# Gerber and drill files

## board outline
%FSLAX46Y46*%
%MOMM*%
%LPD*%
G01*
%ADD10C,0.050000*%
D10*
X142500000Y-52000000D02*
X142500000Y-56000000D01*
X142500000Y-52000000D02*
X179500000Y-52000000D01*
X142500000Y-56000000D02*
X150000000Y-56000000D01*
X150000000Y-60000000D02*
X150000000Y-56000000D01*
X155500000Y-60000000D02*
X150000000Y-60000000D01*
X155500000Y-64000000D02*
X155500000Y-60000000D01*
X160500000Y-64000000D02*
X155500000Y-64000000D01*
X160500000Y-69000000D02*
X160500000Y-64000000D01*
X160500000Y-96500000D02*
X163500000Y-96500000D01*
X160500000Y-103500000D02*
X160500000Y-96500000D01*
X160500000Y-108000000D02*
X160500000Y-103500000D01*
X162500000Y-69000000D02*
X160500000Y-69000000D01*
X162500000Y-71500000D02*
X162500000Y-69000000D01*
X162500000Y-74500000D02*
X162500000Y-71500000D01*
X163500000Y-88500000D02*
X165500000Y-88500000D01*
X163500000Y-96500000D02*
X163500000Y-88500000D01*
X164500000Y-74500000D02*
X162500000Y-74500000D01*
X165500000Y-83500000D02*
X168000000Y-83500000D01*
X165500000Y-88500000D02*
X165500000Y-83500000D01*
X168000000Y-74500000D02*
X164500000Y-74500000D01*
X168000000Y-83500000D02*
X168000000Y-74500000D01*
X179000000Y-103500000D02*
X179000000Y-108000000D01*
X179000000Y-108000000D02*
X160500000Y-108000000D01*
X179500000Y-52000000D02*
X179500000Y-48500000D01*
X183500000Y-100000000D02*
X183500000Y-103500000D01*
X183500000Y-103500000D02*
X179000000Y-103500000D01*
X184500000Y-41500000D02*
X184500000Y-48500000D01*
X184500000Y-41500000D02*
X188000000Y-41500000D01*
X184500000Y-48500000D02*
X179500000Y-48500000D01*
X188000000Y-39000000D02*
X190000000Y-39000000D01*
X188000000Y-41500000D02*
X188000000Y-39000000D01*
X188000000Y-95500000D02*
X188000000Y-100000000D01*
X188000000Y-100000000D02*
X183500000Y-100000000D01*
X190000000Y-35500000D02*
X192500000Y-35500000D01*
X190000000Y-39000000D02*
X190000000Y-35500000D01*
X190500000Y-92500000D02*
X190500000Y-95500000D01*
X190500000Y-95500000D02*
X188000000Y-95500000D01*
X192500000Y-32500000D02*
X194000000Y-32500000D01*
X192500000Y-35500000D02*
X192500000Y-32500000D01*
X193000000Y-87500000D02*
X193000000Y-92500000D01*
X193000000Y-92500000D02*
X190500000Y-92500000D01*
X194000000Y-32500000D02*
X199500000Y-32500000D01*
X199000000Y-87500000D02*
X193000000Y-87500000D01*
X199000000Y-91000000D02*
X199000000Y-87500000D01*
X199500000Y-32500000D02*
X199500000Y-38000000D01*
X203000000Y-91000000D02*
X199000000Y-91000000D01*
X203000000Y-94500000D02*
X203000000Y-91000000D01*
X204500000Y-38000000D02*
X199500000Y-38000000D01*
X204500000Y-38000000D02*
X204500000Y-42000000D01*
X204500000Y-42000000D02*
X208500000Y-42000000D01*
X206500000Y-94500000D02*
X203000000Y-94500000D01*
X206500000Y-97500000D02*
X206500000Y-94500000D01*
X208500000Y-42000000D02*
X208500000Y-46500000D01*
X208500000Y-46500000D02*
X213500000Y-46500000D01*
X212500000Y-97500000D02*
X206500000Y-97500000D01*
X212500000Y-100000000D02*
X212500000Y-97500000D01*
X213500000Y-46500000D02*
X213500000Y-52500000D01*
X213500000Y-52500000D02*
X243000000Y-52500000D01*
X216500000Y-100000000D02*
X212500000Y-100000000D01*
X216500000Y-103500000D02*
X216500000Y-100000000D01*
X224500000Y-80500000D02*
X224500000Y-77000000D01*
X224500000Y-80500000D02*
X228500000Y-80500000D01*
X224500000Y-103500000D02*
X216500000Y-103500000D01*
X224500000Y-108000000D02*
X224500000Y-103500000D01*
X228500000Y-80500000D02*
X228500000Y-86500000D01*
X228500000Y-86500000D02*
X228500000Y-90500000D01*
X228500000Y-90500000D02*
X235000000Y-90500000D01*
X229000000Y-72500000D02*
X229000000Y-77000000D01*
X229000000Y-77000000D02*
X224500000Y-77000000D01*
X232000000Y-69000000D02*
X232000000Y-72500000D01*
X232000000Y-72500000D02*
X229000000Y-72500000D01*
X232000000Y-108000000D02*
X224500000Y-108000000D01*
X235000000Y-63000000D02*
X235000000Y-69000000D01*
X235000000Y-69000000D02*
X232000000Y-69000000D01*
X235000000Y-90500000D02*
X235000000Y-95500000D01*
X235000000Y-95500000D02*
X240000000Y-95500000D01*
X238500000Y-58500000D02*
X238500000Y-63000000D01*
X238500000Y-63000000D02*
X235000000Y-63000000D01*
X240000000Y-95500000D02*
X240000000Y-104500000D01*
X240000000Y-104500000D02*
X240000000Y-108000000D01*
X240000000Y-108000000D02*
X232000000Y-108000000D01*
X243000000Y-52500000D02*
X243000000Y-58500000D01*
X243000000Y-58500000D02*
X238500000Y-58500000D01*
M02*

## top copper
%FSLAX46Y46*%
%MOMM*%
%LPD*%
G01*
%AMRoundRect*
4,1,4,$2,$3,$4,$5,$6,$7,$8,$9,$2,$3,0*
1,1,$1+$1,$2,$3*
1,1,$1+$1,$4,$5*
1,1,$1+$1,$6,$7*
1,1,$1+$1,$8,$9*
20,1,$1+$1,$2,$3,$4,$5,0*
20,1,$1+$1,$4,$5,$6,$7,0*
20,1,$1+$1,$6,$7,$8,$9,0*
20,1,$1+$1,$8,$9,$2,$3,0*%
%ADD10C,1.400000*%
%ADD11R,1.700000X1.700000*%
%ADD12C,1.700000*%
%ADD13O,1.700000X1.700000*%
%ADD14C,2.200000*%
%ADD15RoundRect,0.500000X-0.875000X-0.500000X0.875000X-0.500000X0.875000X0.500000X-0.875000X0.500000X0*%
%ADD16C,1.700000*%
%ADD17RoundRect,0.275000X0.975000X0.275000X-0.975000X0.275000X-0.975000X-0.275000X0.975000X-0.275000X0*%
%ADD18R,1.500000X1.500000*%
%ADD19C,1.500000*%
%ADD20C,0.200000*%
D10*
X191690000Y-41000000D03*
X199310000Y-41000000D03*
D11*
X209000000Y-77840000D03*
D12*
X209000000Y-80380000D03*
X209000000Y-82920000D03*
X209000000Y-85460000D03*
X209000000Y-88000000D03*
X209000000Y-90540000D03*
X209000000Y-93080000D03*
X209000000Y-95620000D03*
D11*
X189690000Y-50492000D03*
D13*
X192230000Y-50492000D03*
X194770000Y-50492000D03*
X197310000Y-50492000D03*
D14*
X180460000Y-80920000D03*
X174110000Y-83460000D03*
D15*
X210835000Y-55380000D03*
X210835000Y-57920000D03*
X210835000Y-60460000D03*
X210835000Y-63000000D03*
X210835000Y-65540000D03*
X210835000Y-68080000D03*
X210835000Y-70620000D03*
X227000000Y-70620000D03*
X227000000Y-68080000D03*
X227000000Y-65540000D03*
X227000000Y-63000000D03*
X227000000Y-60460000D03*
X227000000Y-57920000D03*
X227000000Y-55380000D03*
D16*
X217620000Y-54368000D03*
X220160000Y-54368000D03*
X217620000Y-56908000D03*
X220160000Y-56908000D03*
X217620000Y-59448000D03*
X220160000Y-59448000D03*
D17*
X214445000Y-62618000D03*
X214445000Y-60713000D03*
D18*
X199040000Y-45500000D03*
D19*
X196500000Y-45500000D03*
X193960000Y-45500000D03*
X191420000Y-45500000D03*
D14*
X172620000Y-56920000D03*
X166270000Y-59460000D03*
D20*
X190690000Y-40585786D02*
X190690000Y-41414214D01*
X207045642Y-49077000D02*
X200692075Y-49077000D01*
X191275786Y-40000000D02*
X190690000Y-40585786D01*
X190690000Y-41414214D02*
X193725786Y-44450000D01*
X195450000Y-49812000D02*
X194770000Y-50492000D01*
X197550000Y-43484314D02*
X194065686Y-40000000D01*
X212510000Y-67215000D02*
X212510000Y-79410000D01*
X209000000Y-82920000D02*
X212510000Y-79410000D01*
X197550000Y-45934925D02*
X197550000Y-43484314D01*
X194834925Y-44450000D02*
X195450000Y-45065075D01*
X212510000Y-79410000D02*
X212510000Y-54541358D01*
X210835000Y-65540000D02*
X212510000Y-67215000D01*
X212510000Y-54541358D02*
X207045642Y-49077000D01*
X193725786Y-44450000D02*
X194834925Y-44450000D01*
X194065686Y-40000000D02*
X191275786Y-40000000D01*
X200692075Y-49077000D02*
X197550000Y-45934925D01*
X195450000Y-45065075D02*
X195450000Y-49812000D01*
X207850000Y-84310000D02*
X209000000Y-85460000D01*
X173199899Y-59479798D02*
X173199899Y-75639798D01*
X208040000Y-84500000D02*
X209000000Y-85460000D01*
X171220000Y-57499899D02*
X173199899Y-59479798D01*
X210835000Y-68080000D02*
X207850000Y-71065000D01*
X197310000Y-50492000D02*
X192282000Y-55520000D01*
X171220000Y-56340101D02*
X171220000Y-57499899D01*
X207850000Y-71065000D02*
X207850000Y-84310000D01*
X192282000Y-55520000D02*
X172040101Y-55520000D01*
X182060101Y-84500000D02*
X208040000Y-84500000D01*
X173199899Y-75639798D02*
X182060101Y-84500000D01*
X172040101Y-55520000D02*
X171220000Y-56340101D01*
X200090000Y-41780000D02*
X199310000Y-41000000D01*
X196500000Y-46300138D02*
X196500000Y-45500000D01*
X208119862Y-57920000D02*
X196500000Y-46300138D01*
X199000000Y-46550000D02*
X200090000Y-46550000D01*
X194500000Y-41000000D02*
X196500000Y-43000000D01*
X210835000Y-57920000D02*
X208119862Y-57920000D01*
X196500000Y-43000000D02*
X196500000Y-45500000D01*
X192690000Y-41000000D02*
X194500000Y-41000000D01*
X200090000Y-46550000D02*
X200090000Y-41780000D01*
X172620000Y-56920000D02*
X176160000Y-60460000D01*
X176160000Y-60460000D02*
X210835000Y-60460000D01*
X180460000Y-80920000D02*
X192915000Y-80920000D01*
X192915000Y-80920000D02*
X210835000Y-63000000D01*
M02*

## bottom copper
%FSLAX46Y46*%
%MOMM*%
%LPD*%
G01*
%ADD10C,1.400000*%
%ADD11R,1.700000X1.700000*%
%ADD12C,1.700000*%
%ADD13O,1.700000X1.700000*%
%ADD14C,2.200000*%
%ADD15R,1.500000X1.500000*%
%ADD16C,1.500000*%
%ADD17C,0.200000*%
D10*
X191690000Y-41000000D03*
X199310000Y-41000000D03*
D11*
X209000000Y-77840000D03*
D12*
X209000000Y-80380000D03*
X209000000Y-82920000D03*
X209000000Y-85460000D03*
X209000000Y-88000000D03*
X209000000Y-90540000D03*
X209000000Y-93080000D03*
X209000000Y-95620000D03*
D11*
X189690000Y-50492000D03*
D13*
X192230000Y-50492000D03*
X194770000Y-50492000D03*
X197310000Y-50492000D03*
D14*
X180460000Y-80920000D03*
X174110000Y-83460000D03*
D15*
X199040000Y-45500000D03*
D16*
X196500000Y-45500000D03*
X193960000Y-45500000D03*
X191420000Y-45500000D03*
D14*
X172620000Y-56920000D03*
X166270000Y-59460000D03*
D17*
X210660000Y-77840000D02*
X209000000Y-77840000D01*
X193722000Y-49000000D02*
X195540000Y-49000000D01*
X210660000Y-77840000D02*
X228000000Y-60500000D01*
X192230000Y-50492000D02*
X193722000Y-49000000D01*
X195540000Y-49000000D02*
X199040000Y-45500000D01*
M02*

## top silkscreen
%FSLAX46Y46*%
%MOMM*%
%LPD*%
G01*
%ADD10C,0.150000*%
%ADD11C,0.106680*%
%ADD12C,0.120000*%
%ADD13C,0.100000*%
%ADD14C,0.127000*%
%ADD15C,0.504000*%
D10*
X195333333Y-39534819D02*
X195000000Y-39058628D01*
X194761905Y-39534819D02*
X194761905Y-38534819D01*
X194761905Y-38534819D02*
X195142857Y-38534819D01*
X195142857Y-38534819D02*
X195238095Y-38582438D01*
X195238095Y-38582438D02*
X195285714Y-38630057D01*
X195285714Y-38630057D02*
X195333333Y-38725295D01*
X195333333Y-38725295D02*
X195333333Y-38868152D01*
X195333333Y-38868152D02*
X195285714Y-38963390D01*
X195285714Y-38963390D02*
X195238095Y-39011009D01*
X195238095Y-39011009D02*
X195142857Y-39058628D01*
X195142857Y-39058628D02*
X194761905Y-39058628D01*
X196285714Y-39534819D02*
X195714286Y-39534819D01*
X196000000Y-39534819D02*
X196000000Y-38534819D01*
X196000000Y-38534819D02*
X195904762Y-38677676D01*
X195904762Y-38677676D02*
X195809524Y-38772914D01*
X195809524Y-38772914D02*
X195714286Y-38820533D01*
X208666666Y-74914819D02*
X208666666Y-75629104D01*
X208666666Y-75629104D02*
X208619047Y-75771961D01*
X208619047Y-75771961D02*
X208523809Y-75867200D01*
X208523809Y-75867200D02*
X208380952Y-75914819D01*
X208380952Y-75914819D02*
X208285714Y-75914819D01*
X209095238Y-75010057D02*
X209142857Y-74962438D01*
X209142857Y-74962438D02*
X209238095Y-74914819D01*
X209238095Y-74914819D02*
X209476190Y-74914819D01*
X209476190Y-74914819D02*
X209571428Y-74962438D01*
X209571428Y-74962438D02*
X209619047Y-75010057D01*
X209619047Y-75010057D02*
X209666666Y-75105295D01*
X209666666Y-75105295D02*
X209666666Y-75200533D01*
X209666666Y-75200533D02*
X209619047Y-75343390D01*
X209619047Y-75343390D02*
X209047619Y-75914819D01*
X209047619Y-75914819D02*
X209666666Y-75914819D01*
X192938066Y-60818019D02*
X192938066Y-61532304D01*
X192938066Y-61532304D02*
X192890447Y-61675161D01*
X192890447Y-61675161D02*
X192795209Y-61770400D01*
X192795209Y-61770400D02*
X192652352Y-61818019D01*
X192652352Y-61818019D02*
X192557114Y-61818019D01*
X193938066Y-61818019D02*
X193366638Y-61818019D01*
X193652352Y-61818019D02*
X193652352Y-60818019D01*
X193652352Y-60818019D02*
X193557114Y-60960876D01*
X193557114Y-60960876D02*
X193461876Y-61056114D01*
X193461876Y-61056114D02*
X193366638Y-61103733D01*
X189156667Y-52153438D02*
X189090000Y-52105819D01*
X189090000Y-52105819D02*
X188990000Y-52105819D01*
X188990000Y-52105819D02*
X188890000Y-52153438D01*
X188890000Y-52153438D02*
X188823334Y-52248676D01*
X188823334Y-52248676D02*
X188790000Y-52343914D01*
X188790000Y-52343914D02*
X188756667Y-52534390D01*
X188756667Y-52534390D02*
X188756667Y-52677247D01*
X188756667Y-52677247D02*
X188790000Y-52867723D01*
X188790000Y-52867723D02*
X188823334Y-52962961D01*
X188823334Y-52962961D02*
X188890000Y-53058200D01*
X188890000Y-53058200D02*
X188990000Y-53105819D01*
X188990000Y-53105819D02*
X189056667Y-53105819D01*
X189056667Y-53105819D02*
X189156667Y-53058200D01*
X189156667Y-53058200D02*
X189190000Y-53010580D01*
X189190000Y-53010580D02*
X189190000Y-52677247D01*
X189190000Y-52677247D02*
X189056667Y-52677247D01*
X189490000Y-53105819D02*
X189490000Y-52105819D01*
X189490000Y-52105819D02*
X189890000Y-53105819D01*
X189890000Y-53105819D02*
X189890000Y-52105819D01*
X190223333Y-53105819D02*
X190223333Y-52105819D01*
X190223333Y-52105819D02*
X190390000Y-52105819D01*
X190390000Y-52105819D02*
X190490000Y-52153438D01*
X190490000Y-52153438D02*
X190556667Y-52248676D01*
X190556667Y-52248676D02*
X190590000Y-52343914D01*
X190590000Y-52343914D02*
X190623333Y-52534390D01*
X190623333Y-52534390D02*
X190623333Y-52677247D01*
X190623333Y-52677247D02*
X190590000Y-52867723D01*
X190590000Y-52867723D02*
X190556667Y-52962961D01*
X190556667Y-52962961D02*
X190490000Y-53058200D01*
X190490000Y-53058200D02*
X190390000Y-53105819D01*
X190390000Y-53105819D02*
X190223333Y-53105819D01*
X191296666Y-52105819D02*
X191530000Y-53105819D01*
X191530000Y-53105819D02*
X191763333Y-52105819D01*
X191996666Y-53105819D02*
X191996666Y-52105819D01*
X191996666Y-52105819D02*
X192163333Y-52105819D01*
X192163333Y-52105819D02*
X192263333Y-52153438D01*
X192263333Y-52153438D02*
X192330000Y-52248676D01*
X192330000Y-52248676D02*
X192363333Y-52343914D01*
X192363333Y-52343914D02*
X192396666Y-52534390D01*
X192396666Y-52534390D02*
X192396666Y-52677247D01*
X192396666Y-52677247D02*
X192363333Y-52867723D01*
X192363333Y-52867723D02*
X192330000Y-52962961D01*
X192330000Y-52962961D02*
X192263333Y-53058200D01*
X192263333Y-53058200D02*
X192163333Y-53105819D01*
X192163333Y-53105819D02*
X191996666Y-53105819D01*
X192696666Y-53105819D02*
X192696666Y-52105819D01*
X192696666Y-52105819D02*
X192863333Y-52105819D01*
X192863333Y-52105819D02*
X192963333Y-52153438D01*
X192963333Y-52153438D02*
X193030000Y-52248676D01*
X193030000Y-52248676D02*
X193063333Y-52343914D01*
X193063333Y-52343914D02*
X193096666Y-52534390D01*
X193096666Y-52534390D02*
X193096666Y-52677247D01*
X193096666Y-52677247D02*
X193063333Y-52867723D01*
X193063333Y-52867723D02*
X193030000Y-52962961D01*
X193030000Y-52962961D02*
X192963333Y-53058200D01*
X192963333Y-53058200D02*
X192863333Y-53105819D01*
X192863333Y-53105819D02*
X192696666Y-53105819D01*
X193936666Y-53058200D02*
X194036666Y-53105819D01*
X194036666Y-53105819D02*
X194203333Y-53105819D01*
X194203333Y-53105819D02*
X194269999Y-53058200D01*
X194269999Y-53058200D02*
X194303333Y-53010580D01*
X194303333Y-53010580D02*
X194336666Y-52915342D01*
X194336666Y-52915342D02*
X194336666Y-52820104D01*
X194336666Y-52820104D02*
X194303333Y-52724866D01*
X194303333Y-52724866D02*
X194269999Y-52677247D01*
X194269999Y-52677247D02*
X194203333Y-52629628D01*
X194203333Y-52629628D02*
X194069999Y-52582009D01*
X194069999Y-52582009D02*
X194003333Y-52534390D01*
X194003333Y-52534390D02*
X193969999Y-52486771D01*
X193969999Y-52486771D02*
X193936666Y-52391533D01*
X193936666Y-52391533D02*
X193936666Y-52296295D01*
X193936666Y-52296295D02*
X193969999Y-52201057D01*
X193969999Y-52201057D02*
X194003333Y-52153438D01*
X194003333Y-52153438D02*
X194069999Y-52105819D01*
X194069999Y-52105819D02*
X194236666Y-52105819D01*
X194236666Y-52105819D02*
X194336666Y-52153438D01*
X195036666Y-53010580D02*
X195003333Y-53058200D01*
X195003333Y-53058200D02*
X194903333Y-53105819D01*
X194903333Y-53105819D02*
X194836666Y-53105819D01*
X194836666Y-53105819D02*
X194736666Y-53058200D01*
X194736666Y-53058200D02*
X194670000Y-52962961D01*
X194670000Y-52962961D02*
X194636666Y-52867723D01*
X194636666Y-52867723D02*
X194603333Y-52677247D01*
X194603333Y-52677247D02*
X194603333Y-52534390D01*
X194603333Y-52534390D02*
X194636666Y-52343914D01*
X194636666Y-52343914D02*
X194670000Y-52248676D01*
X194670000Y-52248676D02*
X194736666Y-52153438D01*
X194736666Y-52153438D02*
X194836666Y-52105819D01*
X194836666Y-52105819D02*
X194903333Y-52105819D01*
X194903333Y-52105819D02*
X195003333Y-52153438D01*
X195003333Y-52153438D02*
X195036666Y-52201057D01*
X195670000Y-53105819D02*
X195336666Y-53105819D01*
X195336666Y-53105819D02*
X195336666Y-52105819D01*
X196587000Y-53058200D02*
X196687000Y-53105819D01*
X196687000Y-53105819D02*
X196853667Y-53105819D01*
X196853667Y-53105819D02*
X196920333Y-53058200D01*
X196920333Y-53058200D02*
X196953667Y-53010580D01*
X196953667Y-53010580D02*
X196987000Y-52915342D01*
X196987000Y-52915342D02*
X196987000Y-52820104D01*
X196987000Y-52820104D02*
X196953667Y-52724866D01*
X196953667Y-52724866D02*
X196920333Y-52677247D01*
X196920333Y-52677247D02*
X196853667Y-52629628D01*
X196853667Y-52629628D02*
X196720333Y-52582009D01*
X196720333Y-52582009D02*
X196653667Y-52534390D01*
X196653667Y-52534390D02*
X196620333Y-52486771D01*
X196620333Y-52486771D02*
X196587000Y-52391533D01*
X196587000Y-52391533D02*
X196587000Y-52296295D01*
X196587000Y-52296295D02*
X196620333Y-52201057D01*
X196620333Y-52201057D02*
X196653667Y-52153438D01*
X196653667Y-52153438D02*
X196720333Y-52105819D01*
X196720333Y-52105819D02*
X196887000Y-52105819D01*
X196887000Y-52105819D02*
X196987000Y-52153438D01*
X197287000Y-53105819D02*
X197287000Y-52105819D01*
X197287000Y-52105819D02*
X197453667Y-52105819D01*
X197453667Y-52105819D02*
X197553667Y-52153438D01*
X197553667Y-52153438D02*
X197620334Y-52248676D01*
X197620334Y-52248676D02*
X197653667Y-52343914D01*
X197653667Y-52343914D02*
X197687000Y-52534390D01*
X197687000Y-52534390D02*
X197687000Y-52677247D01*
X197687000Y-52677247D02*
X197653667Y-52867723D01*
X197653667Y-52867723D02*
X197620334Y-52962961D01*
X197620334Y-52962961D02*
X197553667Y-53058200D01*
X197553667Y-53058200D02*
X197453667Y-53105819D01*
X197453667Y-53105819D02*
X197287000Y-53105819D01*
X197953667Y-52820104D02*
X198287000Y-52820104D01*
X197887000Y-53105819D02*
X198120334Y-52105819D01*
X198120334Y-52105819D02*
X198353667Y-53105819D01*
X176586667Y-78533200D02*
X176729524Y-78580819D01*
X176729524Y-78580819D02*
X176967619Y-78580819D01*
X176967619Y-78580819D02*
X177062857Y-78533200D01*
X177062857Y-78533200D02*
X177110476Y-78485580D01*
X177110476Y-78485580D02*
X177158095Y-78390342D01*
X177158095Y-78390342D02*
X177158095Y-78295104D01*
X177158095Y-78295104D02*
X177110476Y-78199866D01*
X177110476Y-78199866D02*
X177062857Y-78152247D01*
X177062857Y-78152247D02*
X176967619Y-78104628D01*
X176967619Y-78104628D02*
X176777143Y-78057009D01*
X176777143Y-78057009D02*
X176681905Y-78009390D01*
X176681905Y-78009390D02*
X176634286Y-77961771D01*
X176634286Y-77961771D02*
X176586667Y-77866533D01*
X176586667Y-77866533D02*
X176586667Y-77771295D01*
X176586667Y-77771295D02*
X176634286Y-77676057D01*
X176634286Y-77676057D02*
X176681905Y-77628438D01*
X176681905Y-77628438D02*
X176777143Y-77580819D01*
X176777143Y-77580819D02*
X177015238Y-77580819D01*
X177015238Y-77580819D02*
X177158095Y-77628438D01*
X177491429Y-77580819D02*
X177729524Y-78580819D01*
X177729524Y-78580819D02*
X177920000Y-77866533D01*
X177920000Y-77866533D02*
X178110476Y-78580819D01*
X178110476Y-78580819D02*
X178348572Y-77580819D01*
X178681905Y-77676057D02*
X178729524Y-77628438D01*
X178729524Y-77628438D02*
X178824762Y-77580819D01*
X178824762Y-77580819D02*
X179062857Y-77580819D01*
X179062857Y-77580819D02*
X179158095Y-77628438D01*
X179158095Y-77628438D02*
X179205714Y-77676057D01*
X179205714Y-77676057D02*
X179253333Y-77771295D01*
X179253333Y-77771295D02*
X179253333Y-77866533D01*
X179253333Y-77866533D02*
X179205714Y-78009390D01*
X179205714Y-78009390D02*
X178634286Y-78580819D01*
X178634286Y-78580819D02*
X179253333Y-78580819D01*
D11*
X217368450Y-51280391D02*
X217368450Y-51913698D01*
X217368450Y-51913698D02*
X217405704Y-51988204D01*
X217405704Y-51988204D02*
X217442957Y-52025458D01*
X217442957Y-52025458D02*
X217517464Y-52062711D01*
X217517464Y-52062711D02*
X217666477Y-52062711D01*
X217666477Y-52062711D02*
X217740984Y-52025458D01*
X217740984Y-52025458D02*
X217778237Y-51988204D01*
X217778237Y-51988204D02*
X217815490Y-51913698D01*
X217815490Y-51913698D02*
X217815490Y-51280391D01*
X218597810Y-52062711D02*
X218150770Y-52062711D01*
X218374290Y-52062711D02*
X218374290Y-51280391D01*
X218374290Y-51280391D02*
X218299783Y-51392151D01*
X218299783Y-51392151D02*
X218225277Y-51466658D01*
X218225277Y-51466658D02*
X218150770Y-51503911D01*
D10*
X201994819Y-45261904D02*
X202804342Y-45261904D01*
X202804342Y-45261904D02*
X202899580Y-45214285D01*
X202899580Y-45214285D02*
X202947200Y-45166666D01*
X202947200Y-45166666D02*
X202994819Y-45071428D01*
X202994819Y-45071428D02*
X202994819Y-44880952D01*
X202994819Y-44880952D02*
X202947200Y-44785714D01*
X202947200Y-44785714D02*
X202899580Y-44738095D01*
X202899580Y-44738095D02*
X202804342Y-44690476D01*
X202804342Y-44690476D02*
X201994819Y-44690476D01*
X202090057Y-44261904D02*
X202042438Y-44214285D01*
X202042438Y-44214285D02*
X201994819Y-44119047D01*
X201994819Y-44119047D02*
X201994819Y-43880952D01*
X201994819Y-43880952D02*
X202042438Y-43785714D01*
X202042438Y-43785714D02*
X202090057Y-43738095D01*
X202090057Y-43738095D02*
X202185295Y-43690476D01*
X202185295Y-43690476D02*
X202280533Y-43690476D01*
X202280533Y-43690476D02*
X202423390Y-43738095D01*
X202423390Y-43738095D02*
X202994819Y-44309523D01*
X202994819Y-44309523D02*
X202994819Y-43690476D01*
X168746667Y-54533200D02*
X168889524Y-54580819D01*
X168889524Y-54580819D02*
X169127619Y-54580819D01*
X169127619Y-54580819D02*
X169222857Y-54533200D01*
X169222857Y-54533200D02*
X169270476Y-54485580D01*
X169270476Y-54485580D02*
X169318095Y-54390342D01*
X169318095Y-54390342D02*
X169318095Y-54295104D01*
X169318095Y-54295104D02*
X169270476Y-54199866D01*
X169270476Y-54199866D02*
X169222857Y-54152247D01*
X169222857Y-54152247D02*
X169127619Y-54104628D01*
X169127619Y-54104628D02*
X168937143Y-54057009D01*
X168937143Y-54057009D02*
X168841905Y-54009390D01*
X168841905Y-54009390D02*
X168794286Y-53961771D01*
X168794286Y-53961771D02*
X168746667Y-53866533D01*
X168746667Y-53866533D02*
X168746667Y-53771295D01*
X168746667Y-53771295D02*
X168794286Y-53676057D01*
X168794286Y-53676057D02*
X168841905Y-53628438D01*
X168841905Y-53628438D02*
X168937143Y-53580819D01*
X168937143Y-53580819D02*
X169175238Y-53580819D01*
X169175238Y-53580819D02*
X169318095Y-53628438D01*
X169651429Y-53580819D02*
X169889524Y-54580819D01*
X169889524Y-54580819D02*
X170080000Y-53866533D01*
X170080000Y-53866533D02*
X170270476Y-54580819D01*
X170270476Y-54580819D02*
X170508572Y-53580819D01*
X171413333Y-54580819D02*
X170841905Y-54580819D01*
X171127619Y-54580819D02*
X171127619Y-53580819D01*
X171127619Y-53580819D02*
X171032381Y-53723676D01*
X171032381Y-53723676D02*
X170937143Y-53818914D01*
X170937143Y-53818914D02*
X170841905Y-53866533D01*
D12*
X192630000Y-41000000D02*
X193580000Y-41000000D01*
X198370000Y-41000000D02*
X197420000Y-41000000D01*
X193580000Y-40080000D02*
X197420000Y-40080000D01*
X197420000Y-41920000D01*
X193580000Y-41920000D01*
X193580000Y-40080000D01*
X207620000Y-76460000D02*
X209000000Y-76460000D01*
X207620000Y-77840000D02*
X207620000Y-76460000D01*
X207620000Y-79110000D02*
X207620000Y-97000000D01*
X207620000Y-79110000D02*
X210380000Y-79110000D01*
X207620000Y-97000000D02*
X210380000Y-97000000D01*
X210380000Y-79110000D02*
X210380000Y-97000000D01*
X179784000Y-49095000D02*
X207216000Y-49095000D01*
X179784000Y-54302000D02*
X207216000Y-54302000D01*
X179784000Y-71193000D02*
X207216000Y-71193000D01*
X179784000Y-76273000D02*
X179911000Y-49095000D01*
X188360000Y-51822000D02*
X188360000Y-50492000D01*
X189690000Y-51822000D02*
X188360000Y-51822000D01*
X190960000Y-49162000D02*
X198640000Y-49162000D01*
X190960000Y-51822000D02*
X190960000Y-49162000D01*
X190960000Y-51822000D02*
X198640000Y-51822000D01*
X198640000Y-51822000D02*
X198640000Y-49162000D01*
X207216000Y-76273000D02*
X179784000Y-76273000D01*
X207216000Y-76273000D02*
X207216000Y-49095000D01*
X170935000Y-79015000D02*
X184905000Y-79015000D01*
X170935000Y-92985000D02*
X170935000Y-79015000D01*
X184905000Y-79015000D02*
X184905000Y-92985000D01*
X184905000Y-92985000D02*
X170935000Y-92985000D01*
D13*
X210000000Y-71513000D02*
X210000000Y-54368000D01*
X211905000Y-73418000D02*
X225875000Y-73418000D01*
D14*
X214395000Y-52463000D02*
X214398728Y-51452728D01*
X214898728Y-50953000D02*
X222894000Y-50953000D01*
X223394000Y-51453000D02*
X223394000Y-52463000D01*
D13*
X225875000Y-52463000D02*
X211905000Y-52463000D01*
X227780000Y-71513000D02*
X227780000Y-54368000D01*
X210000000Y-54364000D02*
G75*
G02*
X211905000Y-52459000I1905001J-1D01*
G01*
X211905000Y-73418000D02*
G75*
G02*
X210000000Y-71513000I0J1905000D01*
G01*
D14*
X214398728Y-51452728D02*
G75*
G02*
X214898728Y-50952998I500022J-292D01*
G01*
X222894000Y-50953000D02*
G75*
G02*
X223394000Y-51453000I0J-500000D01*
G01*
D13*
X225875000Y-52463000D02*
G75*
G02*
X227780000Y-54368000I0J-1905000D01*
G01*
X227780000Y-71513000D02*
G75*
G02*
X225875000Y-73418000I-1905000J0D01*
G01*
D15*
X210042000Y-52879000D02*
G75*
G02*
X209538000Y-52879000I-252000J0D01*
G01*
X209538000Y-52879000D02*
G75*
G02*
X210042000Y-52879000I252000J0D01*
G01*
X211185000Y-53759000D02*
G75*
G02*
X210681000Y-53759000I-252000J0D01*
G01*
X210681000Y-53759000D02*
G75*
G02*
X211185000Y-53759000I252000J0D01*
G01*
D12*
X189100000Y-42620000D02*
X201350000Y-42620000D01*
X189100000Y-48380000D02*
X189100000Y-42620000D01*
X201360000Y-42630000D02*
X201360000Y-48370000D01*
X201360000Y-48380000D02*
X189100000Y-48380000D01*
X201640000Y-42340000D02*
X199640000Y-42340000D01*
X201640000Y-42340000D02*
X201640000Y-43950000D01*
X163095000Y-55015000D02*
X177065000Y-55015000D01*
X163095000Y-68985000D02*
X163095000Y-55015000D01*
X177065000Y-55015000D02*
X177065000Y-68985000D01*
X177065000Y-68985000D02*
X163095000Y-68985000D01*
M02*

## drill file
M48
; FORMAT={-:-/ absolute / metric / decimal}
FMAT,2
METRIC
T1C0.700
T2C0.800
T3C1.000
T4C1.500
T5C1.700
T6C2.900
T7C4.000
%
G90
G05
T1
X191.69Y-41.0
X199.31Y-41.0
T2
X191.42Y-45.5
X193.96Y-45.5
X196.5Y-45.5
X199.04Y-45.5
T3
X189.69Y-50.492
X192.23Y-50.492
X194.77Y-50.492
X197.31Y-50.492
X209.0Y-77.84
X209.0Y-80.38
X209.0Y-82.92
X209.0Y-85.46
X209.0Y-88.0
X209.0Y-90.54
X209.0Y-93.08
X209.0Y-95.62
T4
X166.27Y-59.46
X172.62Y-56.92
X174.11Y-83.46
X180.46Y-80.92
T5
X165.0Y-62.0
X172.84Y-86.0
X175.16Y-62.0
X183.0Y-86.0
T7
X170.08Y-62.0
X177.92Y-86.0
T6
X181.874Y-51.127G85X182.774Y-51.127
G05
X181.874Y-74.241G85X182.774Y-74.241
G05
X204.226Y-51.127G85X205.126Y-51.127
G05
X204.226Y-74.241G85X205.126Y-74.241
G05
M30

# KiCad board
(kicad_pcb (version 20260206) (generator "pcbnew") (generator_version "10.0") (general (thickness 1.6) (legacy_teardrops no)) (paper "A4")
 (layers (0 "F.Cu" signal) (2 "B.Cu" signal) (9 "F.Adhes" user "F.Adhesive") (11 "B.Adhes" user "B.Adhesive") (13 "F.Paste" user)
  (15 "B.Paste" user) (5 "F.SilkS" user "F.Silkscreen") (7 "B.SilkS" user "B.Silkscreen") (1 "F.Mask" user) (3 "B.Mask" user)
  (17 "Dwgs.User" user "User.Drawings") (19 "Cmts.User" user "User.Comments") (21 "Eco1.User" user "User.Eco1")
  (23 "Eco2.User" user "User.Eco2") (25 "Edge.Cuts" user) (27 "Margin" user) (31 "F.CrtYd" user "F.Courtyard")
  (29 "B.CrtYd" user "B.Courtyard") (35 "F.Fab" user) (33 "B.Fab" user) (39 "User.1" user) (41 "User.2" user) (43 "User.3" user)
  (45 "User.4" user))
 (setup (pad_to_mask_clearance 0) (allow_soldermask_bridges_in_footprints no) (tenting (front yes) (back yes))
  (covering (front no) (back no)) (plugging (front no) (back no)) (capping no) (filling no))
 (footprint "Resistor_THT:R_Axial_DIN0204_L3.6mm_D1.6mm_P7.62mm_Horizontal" (layer "F.Cu") (at 191.69 41)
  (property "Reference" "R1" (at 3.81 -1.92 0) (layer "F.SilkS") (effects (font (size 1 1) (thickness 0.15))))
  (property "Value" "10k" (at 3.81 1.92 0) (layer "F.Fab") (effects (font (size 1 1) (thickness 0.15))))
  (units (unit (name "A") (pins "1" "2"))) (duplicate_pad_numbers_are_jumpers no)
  (fp_line (start 0.94 0) (end 1.89 0) (stroke (width 0.12) (type solid)) (layer "F.SilkS"))
  (fp_line (start 6.68 0) (end 5.73 0) (stroke (width 0.12) (type solid)) (layer "F.SilkS"))
  (fp_rect (start 1.89 -0.92) (end 5.73 0.92) (stroke (width 0.12) (type solid)) (fill no) (layer "F.SilkS"))
  (pad "1" thru_hole circle (at 0 0) (size 1.4 1.4) (drill 0.7) (layers "*.Cu" "*.Mask") (remove_unused_layers no) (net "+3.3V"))
  (pad "2" thru_hole circle (at 7.62 0) (size 1.4 1.4) (drill 0.7) (layers "*.Cu" "*.Mask") (remove_unused_layers no) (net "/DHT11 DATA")))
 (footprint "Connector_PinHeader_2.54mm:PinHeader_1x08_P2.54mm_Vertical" (layer "F.Cu") (at 209 77.84)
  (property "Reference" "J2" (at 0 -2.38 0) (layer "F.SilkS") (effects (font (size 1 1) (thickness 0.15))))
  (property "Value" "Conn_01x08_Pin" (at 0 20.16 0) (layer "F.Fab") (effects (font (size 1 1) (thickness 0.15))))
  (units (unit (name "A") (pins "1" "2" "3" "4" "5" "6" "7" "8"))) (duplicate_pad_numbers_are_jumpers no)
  (fp_line (start -1.38 -1.38) (end 0 -1.38) (stroke (width 0.12) (type solid)) (layer "F.SilkS"))
  (fp_line (start -1.38 0) (end -1.38 -1.38) (stroke (width 0.12) (type solid)) (layer "F.SilkS"))
  (fp_line (start -1.38 1.27) (end -1.38 19.16) (stroke (width 0.12) (type solid)) (layer "F.SilkS"))
  (fp_line (start -1.38 1.27) (end 1.38 1.27) (stroke (width 0.12) (type solid)) (layer "F.SilkS"))
  (fp_line (start -1.38 19.16) (end 1.38 19.16) (stroke (width 0.12) (type solid)) (layer "F.SilkS"))
  (fp_line (start 1.38 1.27) (end 1.38 19.16) (stroke (width 0.12) (type solid)) (layer "F.SilkS"))
  (pad "1" thru_hole rect (at 0 0) (size 1.7 1.7) (drill 1) (layers "*.Cu" "*.Mask") (remove_unused_layers no) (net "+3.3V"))
  (pad "2" thru_hole circle (at 0 2.54) (size 1.7 1.7) (drill 1) (layers "*.Cu" "*.Mask") (remove_unused_layers no) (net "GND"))
  (pad "3" thru_hole circle (at 0 5.08) (size 1.7 1.7) (drill 1) (layers "*.Cu" "*.Mask") (remove_unused_layers no) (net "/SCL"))
  (pad "4" thru_hole circle (at 0 7.62) (size 1.7 1.7) (drill 1) (layers "*.Cu" "*.Mask") (remove_unused_layers no) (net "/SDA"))
  (pad "5" thru_hole circle (at 0 10.16) (size 1.7 1.7) (drill 1) (layers "*.Cu" "*.Mask") (remove_unused_layers no)
   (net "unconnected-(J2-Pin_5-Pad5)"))
  (pad "6" thru_hole circle (at 0 12.7) (size 1.7 1.7) (drill 1) (layers "*.Cu" "*.Mask") (remove_unused_layers no)
   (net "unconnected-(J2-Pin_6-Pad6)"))
  (pad "7" thru_hole circle (at 0 15.24) (size 1.7 1.7) (drill 1) (layers "*.Cu" "*.Mask") (remove_unused_layers no)
   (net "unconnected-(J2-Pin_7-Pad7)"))
  (pad "8" thru_hole circle (at 0 17.78) (size 1.7 1.7) (drill 1) (layers "*.Cu" "*.Mask") (remove_unused_layers no)
   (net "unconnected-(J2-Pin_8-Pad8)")))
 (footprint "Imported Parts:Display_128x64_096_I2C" (layer "F.Cu") (at 193.5 50.492)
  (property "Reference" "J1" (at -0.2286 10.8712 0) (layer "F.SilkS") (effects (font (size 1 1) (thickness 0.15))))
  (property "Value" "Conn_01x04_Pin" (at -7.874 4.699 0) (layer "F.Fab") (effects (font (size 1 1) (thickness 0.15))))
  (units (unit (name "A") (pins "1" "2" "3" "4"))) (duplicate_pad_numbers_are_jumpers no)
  (fp_line (start -13.716 -1.397) (end 13.716 -1.397) (stroke (width 0.12) (type solid)) (layer "F.SilkS"))
  (fp_line (start -13.716 3.81) (end 13.716 3.81) (stroke (width 0.12) (type solid)) (layer "F.SilkS"))
  (fp_line (start -13.716 20.701) (end 13.716 20.701) (stroke (width 0.12) (type solid)) (layer "F.SilkS"))
  (fp_line (start -13.716 25.781) (end -13.589 -1.397) (stroke (width 0.12) (type solid)) (layer "F.SilkS"))
  (fp_line (start -5.14 1.33) (end -5.14 0) (stroke (width 0.12) (type solid)) (layer "F.SilkS"))
  (fp_line (start -3.81 1.33) (end -5.14 1.33) (stroke (width 0.12) (type solid)) (layer "F.SilkS"))
  (fp_line (start -2.54 -1.33) (end 5.14 -1.33) (stroke (width 0.12) (type solid)) (layer "F.SilkS"))
  (fp_line (start -2.54 1.33) (end -2.54 -1.33) (stroke (width 0.12) (type solid)) (layer "F.SilkS"))
  (fp_line (start -2.54 1.33) (end 5.14 1.33) (stroke (width 0.12) (type solid)) (layer "F.SilkS"))
  (fp_line (start 5.14 1.33) (end 5.14 -1.33) (stroke (width 0.12) (type solid)) (layer "F.SilkS"))
  (fp_line (start 13.716 25.781) (end -13.716 25.781) (stroke (width 0.12) (type solid)) (layer "F.SilkS"))
  (fp_line (start 13.716 25.781) (end 13.716 -1.397) (stroke (width 0.12) (type solid)) (layer "F.SilkS"))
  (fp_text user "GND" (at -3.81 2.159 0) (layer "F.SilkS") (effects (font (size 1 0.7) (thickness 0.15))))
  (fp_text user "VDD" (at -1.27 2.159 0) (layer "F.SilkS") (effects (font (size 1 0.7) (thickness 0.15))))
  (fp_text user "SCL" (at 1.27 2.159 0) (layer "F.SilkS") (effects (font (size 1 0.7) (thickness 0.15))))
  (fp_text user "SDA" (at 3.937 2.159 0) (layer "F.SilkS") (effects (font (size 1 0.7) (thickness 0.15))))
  (pad "" np_thru_hole oval (at -11.176 0.635) (size 3.8 2.9) (drill oval 3.8 2.9) (layers "*.Cu" "*.Mask"))
  (pad "" np_thru_hole oval (at -11.176 23.749) (size 3.8 2.9) (drill oval 3.8 2.9) (layers "*.Cu" "*.Mask"))
  (pad "" np_thru_hole oval (at 11.176 0.635) (size 3.8 2.9) (drill oval 3.8 2.9) (layers "*.Cu" "*.Mask"))
  (pad "" np_thru_hole oval (at 11.176 23.749) (size 3.8 2.9) (drill oval 3.8 2.9) (layers "*.Cu" "*.Mask"))
  (pad "1" thru_hole rect (at -3.81 0 90) (size 1.7 1.7) (drill 1) (layers "*.Cu" "*.Mask") (remove_unused_layers no) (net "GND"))
  (pad "2" thru_hole oval (at -1.27 0 90) (size 1.7 1.7) (drill 1) (layers "*.Cu" "*.Mask") (remove_unused_layers no) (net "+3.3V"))
  (pad "3" thru_hole oval (at 1.27 0 90) (size 1.7 1.7) (drill 1) (layers "*.Cu" "*.Mask") (remove_unused_layers no) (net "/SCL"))
  (pad "4" thru_hole oval (at 3.81 0 90) (size 1.7 1.7) (drill 1) (layers "*.Cu" "*.Mask") (remove_unused_layers no) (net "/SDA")))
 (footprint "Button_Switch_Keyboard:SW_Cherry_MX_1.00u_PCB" (layer "F.Cu") (at 180.46 80.92)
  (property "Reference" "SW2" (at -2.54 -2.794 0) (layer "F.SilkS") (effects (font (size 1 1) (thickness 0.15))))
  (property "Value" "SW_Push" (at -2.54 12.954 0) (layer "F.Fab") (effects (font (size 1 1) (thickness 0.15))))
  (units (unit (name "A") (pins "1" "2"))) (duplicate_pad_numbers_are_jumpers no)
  (fp_line (start -9.525 -1.905) (end 4.445 -1.905) (stroke (width 0.12) (type solid)) (layer "F.SilkS"))
  (fp_line (start -9.525 12.065) (end -9.525 -1.905) (stroke (width 0.12) (type solid)) (layer "F.SilkS"))
  (fp_line (start 4.445 -1.905) (end 4.445 12.065) (stroke (width 0.12) (type solid)) (layer "F.SilkS"))
  (fp_line (start 4.445 12.065) (end -9.525 12.065) (stroke (width 0.12) (type solid)) (layer "F.SilkS"))
  (pad "" np_thru_hole circle (at -7.62 5.08) (size 1.7 1.7) (drill 1.7) (layers "*.Cu" "*.Mask"))
  (pad "" np_thru_hole circle (at -2.54 5.08) (size 4 4) (drill 4) (layers "*.Cu" "*.Mask"))
  (pad "" np_thru_hole circle (at 2.54 5.08) (size 1.7 1.7) (drill 1.7) (layers "*.Cu" "*.Mask"))
  (pad "1" thru_hole circle (at 0 0) (size 2.2 2.2) (drill 1.5) (layers "*.Cu" "*.Mask") (remove_unused_layers no) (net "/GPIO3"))
  (pad "2" thru_hole circle (at -6.35 2.54) (size 2.2 2.2) (drill 1.5) (layers "*.Cu" "*.Mask") (remove_unused_layers no) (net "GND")))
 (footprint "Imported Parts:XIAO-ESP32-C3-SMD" (layer "F.Cu") (at 210 73.5)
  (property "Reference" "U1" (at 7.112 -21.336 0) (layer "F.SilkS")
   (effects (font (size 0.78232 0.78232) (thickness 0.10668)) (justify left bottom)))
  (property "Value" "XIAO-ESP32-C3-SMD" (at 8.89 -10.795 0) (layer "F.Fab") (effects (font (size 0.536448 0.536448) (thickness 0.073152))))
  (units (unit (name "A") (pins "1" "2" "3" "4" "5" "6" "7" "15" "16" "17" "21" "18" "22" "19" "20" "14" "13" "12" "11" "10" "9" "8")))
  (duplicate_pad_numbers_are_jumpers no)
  (fp_line (start 0 -1.987) (end 0 -19.132) (stroke (width 0.1) (type solid)) (layer "F.SilkS"))
  (fp_line (start 1.905 -0.082) (end 15.875 -0.082) (stroke (width 0.1) (type solid)) (layer "F.SilkS"))
  (fp_line (start 4.395 -21.037) (end 4.398728 -22.047272) (stroke (width 0.127) (type solid)) (layer "F.SilkS"))
  (fp_line (start 4.898728 -22.547) (end 12.894 -22.547) (stroke (width 0.127) (type solid)) (layer "F.SilkS"))
  (fp_line (start 13.394 -22.047) (end 13.394 -21.037) (stroke (width 0.127) (type solid)) (layer "F.SilkS"))
  (fp_line (start 15.875 -21.037) (end 1.905 -21.037) (stroke (width 0.1) (type solid)) (layer "F.SilkS"))
  (fp_line (start 17.78 -1.987) (end 17.78 -19.132) (stroke (width 0.1) (type solid)) (layer "F.SilkS"))
  (fp_arc (start 0 -19.136) (mid 0.557962 -20.483038) (end 1.905 -21.041) (stroke (width 0.1) (type solid)) (layer "F.SilkS"))
  (fp_arc (start 1.905 -0.082) (mid 0.557962 -0.639962) (end 0 -1.987) (stroke (width 0.1) (type solid)) (layer "F.SilkS"))
  (fp_arc (start 4.398728 -22.047272) (mid 4.545272 -22.40064) (end 4.898728 -22.547) (stroke (width 0.127) (type default))
   (layer "F.SilkS"))
  (fp_arc (start 12.894 -22.547) (mid 13.247553 -22.400553) (end 13.394 -22.047) (stroke (width 0.127) (type default)) (layer "F.SilkS"))
  (fp_arc (start 15.875 -21.037) (mid 17.222038 -20.479038) (end 17.78 -19.132) (stroke (width 0.1) (type solid)) (layer "F.SilkS"))
  (fp_arc (start 17.78 -1.987) (mid 17.222038 -0.639962) (end 15.875 -0.082) (stroke (width 0.1) (type solid)) (layer "F.SilkS"))
  (fp_circle (center -0.21 -20.621) (end -0.21 -20.875) (stroke (width 0.5) (type solid)) (fill yes) (layer "F.SilkS"))
  (fp_circle (center 0.933 -19.741) (end 0.933 -19.995) (stroke (width 0.5) (type solid)) (fill yes) (layer "F.SilkS"))
  (pad "1" smd roundrect (at 0.835 -18.12) (size 2.75 2) (layers "F.Cu" "F.Mask" "F.Paste") (roundrect_rratio 0.25)
   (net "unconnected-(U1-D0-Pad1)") (solder_mask_margin 0.0508) (thermal_bridge_angle 45))
  (pad "2" smd roundrect (at 0.835 -15.58) (size 2.75 2) (layers "F.Cu" "F.Mask" "F.Paste") (roundrect_rratio 0.25) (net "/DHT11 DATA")
   (solder_mask_margin 0.0508) (thermal_bridge_angle 45))
  (pad "3" smd roundrect (at 0.835 -13.04) (size 2.75 2) (layers "F.Cu" "F.Mask" "F.Paste") (roundrect_rratio 0.25) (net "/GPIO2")
   (solder_mask_margin 0.0508) (thermal_bridge_angle 45))
  (pad "4" smd roundrect (at 0.835 -10.5) (size 2.75 2) (layers "F.Cu" "F.Mask" "F.Paste") (roundrect_rratio 0.25) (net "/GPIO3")
   (solder_mask_margin 0.0508) (thermal_bridge_angle 45))
  (pad "5" smd roundrect (at 0.835 -7.96) (size 2.75 2) (layers "F.Cu" "F.Mask" "F.Paste") (roundrect_rratio 0.25) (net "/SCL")
   (solder_mask_margin 0.0508) (thermal_bridge_angle 45))
  (pad "6" smd roundrect (at 0.835 -5.42) (size 2.75 2) (layers "F.Cu" "F.Mask" "F.Paste") (roundrect_rratio 0.25) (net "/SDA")
   (solder_mask_margin 0.0508) (thermal_bridge_angle 45))
  (pad "7" smd roundrect (at 0.835 -2.88) (size 2.75 2) (layers "F.Cu" "F.Mask" "F.Paste") (roundrect_rratio 0.25)
   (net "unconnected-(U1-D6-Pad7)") (solder_mask_margin 0.0508) (thermal_bridge_angle 45))
  (pad "8" smd roundrect (at 17 -2.88) (size 2.75 2) (layers "F.Cu" "F.Mask" "F.Paste") (roundrect_rratio 0.25)
   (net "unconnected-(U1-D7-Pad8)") (solder_mask_margin 0.0508) (thermal_bridge_angle 45))
  (pad "9" smd roundrect (at 17 -5.42) (size 2.75 2) (layers "F.Cu" "F.Mask" "F.Paste") (roundrect_rratio 0.25)
   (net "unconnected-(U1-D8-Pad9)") (solder_mask_margin 0.0508) (thermal_bridge_angle 45))
  (pad "10" smd roundrect (at 17 -7.96) (size 2.75 2) (layers "F.Cu" "F.Mask" "F.Paste") (roundrect_rratio 0.25)
   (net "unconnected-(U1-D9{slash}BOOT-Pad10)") (solder_mask_margin 0.0508) (thermal_bridge_angle 45))
  (pad "11" smd roundrect (at 17 -10.5) (size 2.75 2) (layers "F.Cu" "F.Mask" "F.Paste") (roundrect_rratio 0.25)
   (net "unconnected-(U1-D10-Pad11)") (solder_mask_margin 0.0508) (thermal_bridge_angle 45))
  (pad "12" smd roundrect (at 17 -13.04) (size 2.75 2) (layers "F.Cu" "F.Mask" "F.Paste") (roundrect_rratio 0.25) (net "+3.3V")
   (solder_mask_margin 0.0508) (thermal_bridge_angle 45))
  (pad "13" smd roundrect (at 17 -15.58) (size 2.75 2) (layers "F.Cu" "F.Mask" "F.Paste") (roundrect_rratio 0.25) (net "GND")
   (solder_mask_margin 0.0508) (thermal_bridge_angle 45))
  (pad "14" smd roundrect (at 17 -18.12) (size 2.75 2) (layers "F.Cu" "F.Mask" "F.Paste") (roundrect_rratio 0.25) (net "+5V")
   (solder_mask_margin 0.0508) (thermal_bridge_angle 45))
  (pad "15" smd circle (at 7.62 -19.132) (size 1.7 1.7) (layers "F.Cu" "F.Mask" "F.Paste") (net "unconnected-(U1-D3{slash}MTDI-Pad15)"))
  (pad "16" smd circle (at 10.16 -19.132) (size 1.7 1.7) (layers "F.Cu" "F.Mask" "F.Paste") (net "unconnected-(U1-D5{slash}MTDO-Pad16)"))
  (pad "17" smd circle (at 7.62 -16.592) (size 1.7 1.7) (layers "F.Cu" "F.Mask" "F.Paste") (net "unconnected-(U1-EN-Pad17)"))
  (pad "18" smd circle (at 10.16 -16.592) (size 1.7 1.7) (layers "F.Cu" "F.Mask" "F.Paste") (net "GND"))
  (pad "19" smd circle (at 7.62 -14.052) (size 1.7 1.7) (layers "F.Cu" "F.Mask" "F.Paste") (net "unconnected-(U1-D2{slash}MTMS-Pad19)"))
  (pad "20" smd circle (at 10.16 -14.052) (size 1.7 1.7) (layers "F.Cu" "F.Mask" "F.Paste") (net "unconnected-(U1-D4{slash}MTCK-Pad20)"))
  (pad "21" smd roundrect (at 4.445 -10.882 180) (size 2.5 1.1) (layers "F.Cu" "F.Mask" "F.Paste") (roundrect_rratio 0.25)
   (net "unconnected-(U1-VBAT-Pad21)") (thermal_bridge_angle 45))
  (pad "22" smd roundrect (at 4.445 -12.787 180) (size 2.5 1.1) (layers "F.Cu" "F.Mask" "F.Paste") (roundrect_rratio 0.25)
   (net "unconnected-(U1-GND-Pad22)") (thermal_bridge_angle 45)))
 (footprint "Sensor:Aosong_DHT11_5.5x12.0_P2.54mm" (layer "F.Cu") (at 199.04 45.5 -90)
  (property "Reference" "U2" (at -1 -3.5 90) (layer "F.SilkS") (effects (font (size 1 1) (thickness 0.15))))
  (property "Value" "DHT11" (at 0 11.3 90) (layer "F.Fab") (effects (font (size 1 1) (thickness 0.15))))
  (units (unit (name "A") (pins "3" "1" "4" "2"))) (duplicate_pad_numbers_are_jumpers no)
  (fp_line (start -2.88 9.94) (end -2.88 -2.31) (stroke (width 0.12) (type solid)) (layer "F.SilkS"))
  (fp_line (start 2.88 9.94) (end -2.88 9.94) (stroke (width 0.12) (type solid)) (layer "F.SilkS"))
  (fp_line (start -2.87 -2.32) (end 2.87 -2.32) (stroke (width 0.12) (type solid)) (layer "F.SilkS"))
  (fp_line (start 2.88 -2.32) (end 2.88 9.94) (stroke (width 0.12) (type solid)) (layer "F.SilkS"))
  (fp_line (start -3.16 -2.6) (end -3.16 -0.6) (stroke (width 0.12) (type solid)) (layer "F.SilkS"))
  (fp_line (start -3.16 -2.6) (end -1.55 -2.6) (stroke (width 0.12) (type solid)) (layer "F.SilkS"))
  (pad "1" thru_hole rect (at 0 0 270) (size 1.5 1.5) (drill 0.8) (layers "*.Cu" "*.Mask") (remove_unused_layers no) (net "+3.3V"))
  (pad "2" thru_hole circle (at 0 2.54 270) (size 1.5 1.5) (drill 0.8) (layers "*.Cu" "*.Mask") (remove_unused_layers no)
   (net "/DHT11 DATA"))
  (pad "3" thru_hole circle (at 0 5.08 270) (size 1.5 1.5) (drill 0.8) (layers "*.Cu" "*.Mask") (remove_unused_layers no)
   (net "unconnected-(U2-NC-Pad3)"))
  (pad "4" thru_hole circle (at 0 7.62 270) (size 1.5 1.5) (drill 0.8) (layers "*.Cu" "*.Mask") (remove_unused_layers no) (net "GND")))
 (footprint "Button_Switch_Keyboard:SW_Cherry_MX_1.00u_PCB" (layer "F.Cu") (at 172.62 56.92)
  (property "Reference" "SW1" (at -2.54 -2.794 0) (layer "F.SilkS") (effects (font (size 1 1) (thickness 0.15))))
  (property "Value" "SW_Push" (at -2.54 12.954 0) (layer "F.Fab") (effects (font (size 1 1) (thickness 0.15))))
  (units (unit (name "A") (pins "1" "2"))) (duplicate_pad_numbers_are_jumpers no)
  (fp_line (start -9.525 -1.905) (end 4.445 -1.905) (stroke (width 0.12) (type solid)) (layer "F.SilkS"))
  (fp_line (start -9.525 12.065) (end -9.525 -1.905) (stroke (width 0.12) (type solid)) (layer "F.SilkS"))
  (fp_line (start 4.445 -1.905) (end 4.445 12.065) (stroke (width 0.12) (type solid)) (layer "F.SilkS"))
  (fp_line (start 4.445 12.065) (end -9.525 12.065) (stroke (width 0.12) (type solid)) (layer "F.SilkS"))
  (pad "" np_thru_hole circle (at -7.62 5.08) (size 1.7 1.7) (drill 1.7) (layers "*.Cu" "*.Mask"))
  (pad "" np_thru_hole circle (at -2.54 5.08) (size 4 4) (drill 4) (layers "*.Cu" "*.Mask"))
  (pad "" np_thru_hole circle (at 2.54 5.08) (size 1.7 1.7) (drill 1.7) (layers "*.Cu" "*.Mask"))
  (pad "1" thru_hole circle (at 0 0) (size 2.2 2.2) (drill 1.5) (layers "*.Cu" "*.Mask") (remove_unused_layers no) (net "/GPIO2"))
  (pad "2" thru_hole circle (at -6.35 2.54) (size 2.2 2.2) (drill 1.5) (layers "*.Cu" "*.Mask") (remove_unused_layers no) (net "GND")))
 (gr_line (start 142.5 52) (end 142.5 56) (stroke (width 0.05) (type default)) (layer "Edge.Cuts"))
 (gr_line (start 142.5 52) (end 179.5 52) (stroke (width 0.05) (type default)) (layer "Edge.Cuts"))
 (gr_line (start 142.5 56) (end 150 56) (stroke (width 0.05) (type default)) (layer "Edge.Cuts"))
 (gr_line (start 150 60) (end 150 56) (stroke (width 0.05) (type default)) (layer "Edge.Cuts"))
 (gr_line (start 155.5 60) (end 150 60) (stroke (width 0.05) (type default)) (layer "Edge.Cuts"))
 (gr_line (start 155.5 64) (end 155.5 60) (stroke (width 0.05) (type default)) (layer "Edge.Cuts"))
 (gr_line (start 160.5 64) (end 155.5 64) (stroke (width 0.05) (type default)) (layer "Edge.Cuts"))
 (gr_line (start 160.5 69) (end 160.5 64) (stroke (width 0.05) (type default)) (layer "Edge.Cuts"))
 (gr_line (start 160.5 96.5) (end 163.5 96.5) (stroke (width 0.05) (type default)) (layer "Edge.Cuts"))
 (gr_line (start 160.5 103.5) (end 160.5 96.5) (stroke (width 0.05) (type default)) (layer "Edge.Cuts"))
 (gr_line (start 160.5 108) (end 160.5 103.5) (stroke (width 0.05) (type default)) (layer "Edge.Cuts"))
 (gr_line (start 162.5 69) (end 160.5 69) (stroke (width 0.05) (type default)) (layer "Edge.Cuts"))
 (gr_line (start 162.5 71.5) (end 162.5 69) (stroke (width 0.05) (type default)) (layer "Edge.Cuts"))
 (gr_line (start 162.5 74.5) (end 162.5 71.5) (stroke (width 0.05) (type default)) (layer "Edge.Cuts"))
 (gr_line (start 163.5 88.5) (end 165.5 88.5) (stroke (width 0.05) (type default)) (layer "Edge.Cuts"))
 (gr_line (start 163.5 96.5) (end 163.5 88.5) (stroke (width 0.05) (type default)) (layer "Edge.Cuts"))
 (gr_line (start 164.5 74.5) (end 162.5 74.5) (stroke (width 0.05) (type default)) (layer "Edge.Cuts"))
 (gr_line (start 165.5 83.5) (end 168 83.5) (stroke (width 0.05) (type default)) (layer "Edge.Cuts"))
 (gr_line (start 165.5 88.5) (end 165.5 83.5) (stroke (width 0.05) (type default)) (layer "Edge.Cuts"))
 (gr_line (start 168 74.5) (end 164.5 74.5) (stroke (width 0.05) (type default)) (layer "Edge.Cuts"))
 (gr_line (start 168 83.5) (end 168 74.5) (stroke (width 0.05) (type default)) (layer "Edge.Cuts"))
 (gr_line (start 179 103.5) (end 179 108) (stroke (width 0.05) (type default)) (layer "Edge.Cuts"))
 (gr_line (start 179 108) (end 160.5 108) (stroke (width 0.05) (type default)) (layer "Edge.Cuts"))
 (gr_line (start 179.5 52) (end 179.5 48.5) (stroke (width 0.05) (type default)) (layer "Edge.Cuts"))
 (gr_line (start 183.5 100) (end 183.5 103.5) (stroke (width 0.05) (type default)) (layer "Edge.Cuts"))
 (gr_line (start 183.5 103.5) (end 179 103.5) (stroke (width 0.05) (type default)) (layer "Edge.Cuts"))
 (gr_line (start 184.5 41.5) (end 184.5 48.5) (stroke (width 0.05) (type default)) (layer "Edge.Cuts"))
 (gr_line (start 184.5 41.5) (end 188 41.5) (stroke (width 0.05) (type default)) (layer "Edge.Cuts"))
 (gr_line (start 184.5 48.5) (end 179.5 48.5) (stroke (width 0.05) (type default)) (layer "Edge.Cuts"))
 (gr_line (start 188 39) (end 190 39) (stroke (width 0.05) (type default)) (layer "Edge.Cuts"))
 (gr_line (start 188 41.5) (end 188 39) (stroke (width 0.05) (type default)) (layer "Edge.Cuts"))
 (gr_line (start 188 95.5) (end 188 100) (stroke (width 0.05) (type default)) (layer "Edge.Cuts"))
 (gr_line (start 188 100) (end 183.5 100) (stroke (width 0.05) (type default)) (layer "Edge.Cuts"))
 (gr_line (start 190 35.5) (end 192.5 35.5) (stroke (width 0.05) (type default)) (layer "Edge.Cuts"))
 (gr_line (start 190 39) (end 190 35.5) (stroke (width 0.05) (type default)) (layer "Edge.Cuts"))
 (gr_line (start 190.5 92.5) (end 190.5 95.5) (stroke (width 0.05) (type default)) (layer "Edge.Cuts"))
 (gr_line (start 190.5 95.5) (end 188 95.5) (stroke (width 0.05) (type default)) (layer "Edge.Cuts"))
 (gr_line (start 192.5 32.5) (end 194 32.5) (stroke (width 0.05) (type default)) (layer "Edge.Cuts"))
 (gr_line (start 192.5 35.5) (end 192.5 32.5) (stroke (width 0.05) (type default)) (layer "Edge.Cuts"))
 (gr_line (start 193 87.5) (end 193 92.5) (stroke (width 0.05) (type default)) (layer "Edge.Cuts"))
 (gr_line (start 193 92.5) (end 190.5 92.5) (stroke (width 0.05) (type default)) (layer "Edge.Cuts"))
 (gr_line (start 194 32.5) (end 199.5 32.5) (stroke (width 0.05) (type default)) (layer "Edge.Cuts"))
 (gr_line (start 199 87.5) (end 193 87.5) (stroke (width 0.05) (type default)) (layer "Edge.Cuts"))
 (gr_line (start 199 91) (end 199 87.5) (stroke (width 0.05) (type default)) (layer "Edge.Cuts"))
 (gr_line (start 199.5 32.5) (end 199.5 38) (stroke (width 0.05) (type default)) (layer "Edge.Cuts"))
 (gr_line (start 203 91) (end 199 91) (stroke (width 0.05) (type default)) (layer "Edge.Cuts"))
 (gr_line (start 203 94.5) (end 203 91) (stroke (width 0.05) (type default)) (layer "Edge.Cuts"))
 (gr_line (start 204.5 38) (end 199.5 38) (stroke (width 0.05) (type default)) (layer "Edge.Cuts"))
 (gr_line (start 204.5 38) (end 204.5 42) (stroke (width 0.05) (type default)) (layer "Edge.Cuts"))
 (gr_line (start 204.5 42) (end 208.5 42) (stroke (width 0.05) (type default)) (layer "Edge.Cuts"))
 (gr_line (start 206.5 94.5) (end 203 94.5) (stroke (width 0.05) (type default)) (layer "Edge.Cuts"))
 (gr_line (start 206.5 97.5) (end 206.5 94.5) (stroke (width 0.05) (type default)) (layer "Edge.Cuts"))
 (gr_line (start 208.5 42) (end 208.5 46.5) (stroke (width 0.05) (type default)) (layer "Edge.Cuts"))
 (gr_line (start 208.5 46.5) (end 213.5 46.5) (stroke (width 0.05) (type default)) (layer "Edge.Cuts"))
 (gr_line (start 212.5 97.5) (end 206.5 97.5) (stroke (width 0.05) (type default)) (layer "Edge.Cuts"))
 (gr_line (start 212.5 100) (end 212.5 97.5) (stroke (width 0.05) (type default)) (layer "Edge.Cuts"))
 (gr_line (start 213.5 46.5) (end 213.5 52.5) (stroke (width 0.05) (type default)) (layer "Edge.Cuts"))
 (gr_line (start 213.5 52.5) (end 243 52.5) (stroke (width 0.05) (type default)) (layer "Edge.Cuts"))
 (gr_line (start 216.5 100) (end 212.5 100) (stroke (width 0.05) (type default)) (layer "Edge.Cuts"))
 (gr_line (start 216.5 103.5) (end 216.5 100) (stroke (width 0.05) (type default)) (layer "Edge.Cuts"))
 (gr_line (start 224.5 80.5) (end 224.5 77) (stroke (width 0.05) (type default)) (layer "Edge.Cuts"))
 (gr_line (start 224.5 80.5) (end 228.5 80.5) (stroke (width 0.05) (type default)) (layer "Edge.Cuts"))
 (gr_line (start 224.5 103.5) (end 216.5 103.5) (stroke (width 0.05) (type default)) (layer "Edge.Cuts"))
 (gr_line (start 224.5 108) (end 224.5 103.5) (stroke (width 0.05) (type default)) (layer "Edge.Cuts"))
 (gr_line (start 228.5 80.5) (end 228.5 86.5) (stroke (width 0.05) (type default)) (layer "Edge.Cuts"))
 (gr_line (start 228.5 86.5) (end 228.5 90.5) (stroke (width 0.05) (type default)) (layer "Edge.Cuts"))
 (gr_line (start 228.5 90.5) (end 235 90.5) (stroke (width 0.05) (type default)) (layer "Edge.Cuts"))
 (gr_line (start 229 72.5) (end 229 77) (stroke (width 0.05) (type default)) (layer "Edge.Cuts"))
 (gr_line (start 229 77) (end 224.5 77) (stroke (width 0.05) (type default)) (layer "Edge.Cuts"))
 (gr_line (start 232 69) (end 232 72.5) (stroke (width 0.05) (type default)) (layer "Edge.Cuts"))
 (gr_line (start 232 72.5) (end 229 72.5) (stroke (width 0.05) (type default)) (layer "Edge.Cuts"))
 (gr_line (start 232 108) (end 224.5 108) (stroke (width 0.05) (type default)) (layer "Edge.Cuts"))
 (gr_line (start 235 63) (end 235 69) (stroke (width 0.05) (type default)) (layer "Edge.Cuts"))
 (gr_line (start 235 69) (end 232 69) (stroke (width 0.05) (type default)) (layer "Edge.Cuts"))
 (gr_line (start 235 90.5) (end 235 95.5) (stroke (width 0.05) (type default)) (layer "Edge.Cuts"))
 (gr_line (start 235 95.5) (end 240 95.5) (stroke (width 0.05) (type default)) (layer "Edge.Cuts"))
 (gr_line (start 238.5 58.5) (end 238.5 63) (stroke (width 0.05) (type default)) (layer "Edge.Cuts"))
 (gr_line (start 238.5 63) (end 235 63) (stroke (width 0.05) (type default)) (layer "Edge.Cuts"))
 (gr_line (start 240 95.5) (end 240 104.5) (stroke (width 0.05) (type default)) (layer "Edge.Cuts"))
 (gr_line (start 240 104.5) (end 240 108) (stroke (width 0.05) (type default)) (layer "Edge.Cuts"))
 (gr_line (start 240 108) (end 232 108) (stroke (width 0.05) (type default)) (layer "Edge.Cuts"))
 (gr_line (start 243 52.5) (end 243 58.5) (stroke (width 0.05) (type default)) (layer "Edge.Cuts"))
 (gr_line (start 243 58.5) (end 238.5 58.5) (stroke (width 0.05) (type default)) (layer "Edge.Cuts"))
 (segment (start 190.69 40.585786) (end 190.69 41.414214) (width 0.2) (layer "F.Cu") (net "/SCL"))
 (segment (start 207.045642 49.077) (end 200.692075 49.077) (width 0.2) (layer "F.Cu") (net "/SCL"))
 (segment (start 191.275786 40) (end 190.69 40.585786) (width 0.2) (layer "F.Cu") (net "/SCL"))
 (segment (start 190.69 41.414214) (end 193.725786 44.45) (width 0.2) (layer "F.Cu") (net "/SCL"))
 (segment (start 195.45 49.812) (end 194.77 50.492) (width 0.2) (layer "F.Cu") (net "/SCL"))
 (segment (start 197.55 43.484314) (end 194.065686 40) (width 0.2) (layer "F.Cu") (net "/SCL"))
 (segment (start 212.51 67.215) (end 212.51 79.41) (width 0.2) (layer "F.Cu") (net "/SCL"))
 (segment (start 209 82.92) (end 212.51 79.41) (width 0.2) (layer "F.Cu") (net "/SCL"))
 (segment (start 197.55 45.934925) (end 197.55 43.484314) (width 0.2) (layer "F.Cu") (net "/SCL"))
 (segment (start 194.834925 44.45) (end 195.45 45.065075) (width 0.2) (layer "F.Cu") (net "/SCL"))
 (segment (start 212.51 79.41) (end 212.51 54.541358) (width 0.2) (layer "F.Cu") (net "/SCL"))
 (segment (start 210.835 65.54) (end 212.51 67.215) (width 0.2) (layer "F.Cu") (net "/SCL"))
 (segment (start 212.51 54.541358) (end 207.045642 49.077) (width 0.2) (layer "F.Cu") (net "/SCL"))
 (segment (start 193.725786 44.45) (end 194.834925 44.45) (width 0.2) (layer "F.Cu") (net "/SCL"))
 (segment (start 194.065686 40) (end 191.275786 40) (width 0.2) (layer "F.Cu") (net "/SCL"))
 (segment (start 200.692075 49.077) (end 197.55 45.934925) (width 0.2) (layer "F.Cu") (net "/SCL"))
 (segment (start 195.45 45.065075) (end 195.45 49.812) (width 0.2) (layer "F.Cu") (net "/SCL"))
 (segment (start 210.66 77.84) (end 209 77.84) (width 0.2) (layer "B.Cu") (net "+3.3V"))
 (segment (start 193.722 49) (end 195.54 49) (width 0.2) (layer "B.Cu") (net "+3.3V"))
 (segment (start 210.66 77.84) (end 228 60.5) (width 0.2) (layer "B.Cu") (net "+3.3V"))
 (segment (start 192.23 50.492) (end 193.722 49) (width 0.2) (layer "B.Cu") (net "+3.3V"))
 (segment (start 195.54 49) (end 199.04 45.5) (width 0.2) (layer "B.Cu") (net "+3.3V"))
 (segment (start 207.85 84.31) (end 209 85.46) (width 0.2) (layer "F.Cu") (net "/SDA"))
 (segment (start 173.199899 59.479798) (end 173.199899 75.639798) (width 0.2) (layer "F.Cu") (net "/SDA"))
 (segment (start 208.04 84.5) (end 209 85.46) (width 0.2) (layer "F.Cu") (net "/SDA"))
 (segment (start 171.22 57.499899) (end 173.199899 59.479798) (width 0.2) (layer "F.Cu") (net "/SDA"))
 (segment (start 210.835 68.08) (end 207.85 71.065) (width 0.2) (layer "F.Cu") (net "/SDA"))
 (segment (start 197.31 50.492) (end 192.282 55.52) (width 0.2) (layer "F.Cu") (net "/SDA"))
 (segment (start 171.22 56.340101) (end 171.22 57.499899) (width 0.2) (layer "F.Cu") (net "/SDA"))
 (segment (start 207.85 71.065) (end 207.85 84.31) (width 0.2) (layer "F.Cu") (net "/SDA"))
 (segment (start 192.282 55.52) (end 172.040101 55.52) (width 0.2) (layer "F.Cu") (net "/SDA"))
 (segment (start 182.060101 84.5) (end 208.04 84.5) (width 0.2) (layer "F.Cu") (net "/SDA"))
 (segment (start 173.199899 75.639798) (end 182.060101 84.5) (width 0.2) (layer "F.Cu") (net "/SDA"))
 (segment (start 172.040101 55.52) (end 171.22 56.340101) (width 0.2) (layer "F.Cu") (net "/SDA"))
 (segment (start 200.09 41.78) (end 199.31 41) (width 0.2) (layer "F.Cu") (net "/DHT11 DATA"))
 (segment (start 196.5 46.300138) (end 196.5 45.5) (width 0.2) (layer "F.Cu") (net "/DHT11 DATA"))
 (segment (start 208.119862 57.92) (end 196.5 46.300138) (width 0.2) (layer "F.Cu") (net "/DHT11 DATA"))
 (segment (start 199 46.55) (end 200.09 46.55) (width 0.2) (layer "F.Cu") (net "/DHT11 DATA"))
 (segment (start 194.5 41) (end 196.5 43) (width 0.2) (layer "F.Cu") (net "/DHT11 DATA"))
 (segment (start 210.835 57.92) (end 208.119862 57.92) (width 0.2) (layer "F.Cu") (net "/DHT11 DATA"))
 (segment (start 196.5 43) (end 196.5 45.5) (width 0.2) (layer "F.Cu") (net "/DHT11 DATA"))
 (segment (start 192.69 41) (end 194.5 41) (width 0.2) (layer "F.Cu") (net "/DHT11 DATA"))
 (segment (start 200.09 46.55) (end 200.09 41.78) (width 0.2) (layer "F.Cu") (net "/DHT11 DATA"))
 (segment (start 172.62 56.92) (end 176.16 60.46) (width 0.2) (layer "F.Cu") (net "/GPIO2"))
 (segment (start 176.16 60.46) (end 210.835 60.46) (width 0.2) (layer "F.Cu") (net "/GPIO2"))
 (segment (start 180.46 80.92) (end 192.915 80.92) (width 0.2) (layer "F.Cu") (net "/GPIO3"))
 (segment (start 192.915 80.92) (end 210.835 63) (width 0.2) (layer "F.Cu") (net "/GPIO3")))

